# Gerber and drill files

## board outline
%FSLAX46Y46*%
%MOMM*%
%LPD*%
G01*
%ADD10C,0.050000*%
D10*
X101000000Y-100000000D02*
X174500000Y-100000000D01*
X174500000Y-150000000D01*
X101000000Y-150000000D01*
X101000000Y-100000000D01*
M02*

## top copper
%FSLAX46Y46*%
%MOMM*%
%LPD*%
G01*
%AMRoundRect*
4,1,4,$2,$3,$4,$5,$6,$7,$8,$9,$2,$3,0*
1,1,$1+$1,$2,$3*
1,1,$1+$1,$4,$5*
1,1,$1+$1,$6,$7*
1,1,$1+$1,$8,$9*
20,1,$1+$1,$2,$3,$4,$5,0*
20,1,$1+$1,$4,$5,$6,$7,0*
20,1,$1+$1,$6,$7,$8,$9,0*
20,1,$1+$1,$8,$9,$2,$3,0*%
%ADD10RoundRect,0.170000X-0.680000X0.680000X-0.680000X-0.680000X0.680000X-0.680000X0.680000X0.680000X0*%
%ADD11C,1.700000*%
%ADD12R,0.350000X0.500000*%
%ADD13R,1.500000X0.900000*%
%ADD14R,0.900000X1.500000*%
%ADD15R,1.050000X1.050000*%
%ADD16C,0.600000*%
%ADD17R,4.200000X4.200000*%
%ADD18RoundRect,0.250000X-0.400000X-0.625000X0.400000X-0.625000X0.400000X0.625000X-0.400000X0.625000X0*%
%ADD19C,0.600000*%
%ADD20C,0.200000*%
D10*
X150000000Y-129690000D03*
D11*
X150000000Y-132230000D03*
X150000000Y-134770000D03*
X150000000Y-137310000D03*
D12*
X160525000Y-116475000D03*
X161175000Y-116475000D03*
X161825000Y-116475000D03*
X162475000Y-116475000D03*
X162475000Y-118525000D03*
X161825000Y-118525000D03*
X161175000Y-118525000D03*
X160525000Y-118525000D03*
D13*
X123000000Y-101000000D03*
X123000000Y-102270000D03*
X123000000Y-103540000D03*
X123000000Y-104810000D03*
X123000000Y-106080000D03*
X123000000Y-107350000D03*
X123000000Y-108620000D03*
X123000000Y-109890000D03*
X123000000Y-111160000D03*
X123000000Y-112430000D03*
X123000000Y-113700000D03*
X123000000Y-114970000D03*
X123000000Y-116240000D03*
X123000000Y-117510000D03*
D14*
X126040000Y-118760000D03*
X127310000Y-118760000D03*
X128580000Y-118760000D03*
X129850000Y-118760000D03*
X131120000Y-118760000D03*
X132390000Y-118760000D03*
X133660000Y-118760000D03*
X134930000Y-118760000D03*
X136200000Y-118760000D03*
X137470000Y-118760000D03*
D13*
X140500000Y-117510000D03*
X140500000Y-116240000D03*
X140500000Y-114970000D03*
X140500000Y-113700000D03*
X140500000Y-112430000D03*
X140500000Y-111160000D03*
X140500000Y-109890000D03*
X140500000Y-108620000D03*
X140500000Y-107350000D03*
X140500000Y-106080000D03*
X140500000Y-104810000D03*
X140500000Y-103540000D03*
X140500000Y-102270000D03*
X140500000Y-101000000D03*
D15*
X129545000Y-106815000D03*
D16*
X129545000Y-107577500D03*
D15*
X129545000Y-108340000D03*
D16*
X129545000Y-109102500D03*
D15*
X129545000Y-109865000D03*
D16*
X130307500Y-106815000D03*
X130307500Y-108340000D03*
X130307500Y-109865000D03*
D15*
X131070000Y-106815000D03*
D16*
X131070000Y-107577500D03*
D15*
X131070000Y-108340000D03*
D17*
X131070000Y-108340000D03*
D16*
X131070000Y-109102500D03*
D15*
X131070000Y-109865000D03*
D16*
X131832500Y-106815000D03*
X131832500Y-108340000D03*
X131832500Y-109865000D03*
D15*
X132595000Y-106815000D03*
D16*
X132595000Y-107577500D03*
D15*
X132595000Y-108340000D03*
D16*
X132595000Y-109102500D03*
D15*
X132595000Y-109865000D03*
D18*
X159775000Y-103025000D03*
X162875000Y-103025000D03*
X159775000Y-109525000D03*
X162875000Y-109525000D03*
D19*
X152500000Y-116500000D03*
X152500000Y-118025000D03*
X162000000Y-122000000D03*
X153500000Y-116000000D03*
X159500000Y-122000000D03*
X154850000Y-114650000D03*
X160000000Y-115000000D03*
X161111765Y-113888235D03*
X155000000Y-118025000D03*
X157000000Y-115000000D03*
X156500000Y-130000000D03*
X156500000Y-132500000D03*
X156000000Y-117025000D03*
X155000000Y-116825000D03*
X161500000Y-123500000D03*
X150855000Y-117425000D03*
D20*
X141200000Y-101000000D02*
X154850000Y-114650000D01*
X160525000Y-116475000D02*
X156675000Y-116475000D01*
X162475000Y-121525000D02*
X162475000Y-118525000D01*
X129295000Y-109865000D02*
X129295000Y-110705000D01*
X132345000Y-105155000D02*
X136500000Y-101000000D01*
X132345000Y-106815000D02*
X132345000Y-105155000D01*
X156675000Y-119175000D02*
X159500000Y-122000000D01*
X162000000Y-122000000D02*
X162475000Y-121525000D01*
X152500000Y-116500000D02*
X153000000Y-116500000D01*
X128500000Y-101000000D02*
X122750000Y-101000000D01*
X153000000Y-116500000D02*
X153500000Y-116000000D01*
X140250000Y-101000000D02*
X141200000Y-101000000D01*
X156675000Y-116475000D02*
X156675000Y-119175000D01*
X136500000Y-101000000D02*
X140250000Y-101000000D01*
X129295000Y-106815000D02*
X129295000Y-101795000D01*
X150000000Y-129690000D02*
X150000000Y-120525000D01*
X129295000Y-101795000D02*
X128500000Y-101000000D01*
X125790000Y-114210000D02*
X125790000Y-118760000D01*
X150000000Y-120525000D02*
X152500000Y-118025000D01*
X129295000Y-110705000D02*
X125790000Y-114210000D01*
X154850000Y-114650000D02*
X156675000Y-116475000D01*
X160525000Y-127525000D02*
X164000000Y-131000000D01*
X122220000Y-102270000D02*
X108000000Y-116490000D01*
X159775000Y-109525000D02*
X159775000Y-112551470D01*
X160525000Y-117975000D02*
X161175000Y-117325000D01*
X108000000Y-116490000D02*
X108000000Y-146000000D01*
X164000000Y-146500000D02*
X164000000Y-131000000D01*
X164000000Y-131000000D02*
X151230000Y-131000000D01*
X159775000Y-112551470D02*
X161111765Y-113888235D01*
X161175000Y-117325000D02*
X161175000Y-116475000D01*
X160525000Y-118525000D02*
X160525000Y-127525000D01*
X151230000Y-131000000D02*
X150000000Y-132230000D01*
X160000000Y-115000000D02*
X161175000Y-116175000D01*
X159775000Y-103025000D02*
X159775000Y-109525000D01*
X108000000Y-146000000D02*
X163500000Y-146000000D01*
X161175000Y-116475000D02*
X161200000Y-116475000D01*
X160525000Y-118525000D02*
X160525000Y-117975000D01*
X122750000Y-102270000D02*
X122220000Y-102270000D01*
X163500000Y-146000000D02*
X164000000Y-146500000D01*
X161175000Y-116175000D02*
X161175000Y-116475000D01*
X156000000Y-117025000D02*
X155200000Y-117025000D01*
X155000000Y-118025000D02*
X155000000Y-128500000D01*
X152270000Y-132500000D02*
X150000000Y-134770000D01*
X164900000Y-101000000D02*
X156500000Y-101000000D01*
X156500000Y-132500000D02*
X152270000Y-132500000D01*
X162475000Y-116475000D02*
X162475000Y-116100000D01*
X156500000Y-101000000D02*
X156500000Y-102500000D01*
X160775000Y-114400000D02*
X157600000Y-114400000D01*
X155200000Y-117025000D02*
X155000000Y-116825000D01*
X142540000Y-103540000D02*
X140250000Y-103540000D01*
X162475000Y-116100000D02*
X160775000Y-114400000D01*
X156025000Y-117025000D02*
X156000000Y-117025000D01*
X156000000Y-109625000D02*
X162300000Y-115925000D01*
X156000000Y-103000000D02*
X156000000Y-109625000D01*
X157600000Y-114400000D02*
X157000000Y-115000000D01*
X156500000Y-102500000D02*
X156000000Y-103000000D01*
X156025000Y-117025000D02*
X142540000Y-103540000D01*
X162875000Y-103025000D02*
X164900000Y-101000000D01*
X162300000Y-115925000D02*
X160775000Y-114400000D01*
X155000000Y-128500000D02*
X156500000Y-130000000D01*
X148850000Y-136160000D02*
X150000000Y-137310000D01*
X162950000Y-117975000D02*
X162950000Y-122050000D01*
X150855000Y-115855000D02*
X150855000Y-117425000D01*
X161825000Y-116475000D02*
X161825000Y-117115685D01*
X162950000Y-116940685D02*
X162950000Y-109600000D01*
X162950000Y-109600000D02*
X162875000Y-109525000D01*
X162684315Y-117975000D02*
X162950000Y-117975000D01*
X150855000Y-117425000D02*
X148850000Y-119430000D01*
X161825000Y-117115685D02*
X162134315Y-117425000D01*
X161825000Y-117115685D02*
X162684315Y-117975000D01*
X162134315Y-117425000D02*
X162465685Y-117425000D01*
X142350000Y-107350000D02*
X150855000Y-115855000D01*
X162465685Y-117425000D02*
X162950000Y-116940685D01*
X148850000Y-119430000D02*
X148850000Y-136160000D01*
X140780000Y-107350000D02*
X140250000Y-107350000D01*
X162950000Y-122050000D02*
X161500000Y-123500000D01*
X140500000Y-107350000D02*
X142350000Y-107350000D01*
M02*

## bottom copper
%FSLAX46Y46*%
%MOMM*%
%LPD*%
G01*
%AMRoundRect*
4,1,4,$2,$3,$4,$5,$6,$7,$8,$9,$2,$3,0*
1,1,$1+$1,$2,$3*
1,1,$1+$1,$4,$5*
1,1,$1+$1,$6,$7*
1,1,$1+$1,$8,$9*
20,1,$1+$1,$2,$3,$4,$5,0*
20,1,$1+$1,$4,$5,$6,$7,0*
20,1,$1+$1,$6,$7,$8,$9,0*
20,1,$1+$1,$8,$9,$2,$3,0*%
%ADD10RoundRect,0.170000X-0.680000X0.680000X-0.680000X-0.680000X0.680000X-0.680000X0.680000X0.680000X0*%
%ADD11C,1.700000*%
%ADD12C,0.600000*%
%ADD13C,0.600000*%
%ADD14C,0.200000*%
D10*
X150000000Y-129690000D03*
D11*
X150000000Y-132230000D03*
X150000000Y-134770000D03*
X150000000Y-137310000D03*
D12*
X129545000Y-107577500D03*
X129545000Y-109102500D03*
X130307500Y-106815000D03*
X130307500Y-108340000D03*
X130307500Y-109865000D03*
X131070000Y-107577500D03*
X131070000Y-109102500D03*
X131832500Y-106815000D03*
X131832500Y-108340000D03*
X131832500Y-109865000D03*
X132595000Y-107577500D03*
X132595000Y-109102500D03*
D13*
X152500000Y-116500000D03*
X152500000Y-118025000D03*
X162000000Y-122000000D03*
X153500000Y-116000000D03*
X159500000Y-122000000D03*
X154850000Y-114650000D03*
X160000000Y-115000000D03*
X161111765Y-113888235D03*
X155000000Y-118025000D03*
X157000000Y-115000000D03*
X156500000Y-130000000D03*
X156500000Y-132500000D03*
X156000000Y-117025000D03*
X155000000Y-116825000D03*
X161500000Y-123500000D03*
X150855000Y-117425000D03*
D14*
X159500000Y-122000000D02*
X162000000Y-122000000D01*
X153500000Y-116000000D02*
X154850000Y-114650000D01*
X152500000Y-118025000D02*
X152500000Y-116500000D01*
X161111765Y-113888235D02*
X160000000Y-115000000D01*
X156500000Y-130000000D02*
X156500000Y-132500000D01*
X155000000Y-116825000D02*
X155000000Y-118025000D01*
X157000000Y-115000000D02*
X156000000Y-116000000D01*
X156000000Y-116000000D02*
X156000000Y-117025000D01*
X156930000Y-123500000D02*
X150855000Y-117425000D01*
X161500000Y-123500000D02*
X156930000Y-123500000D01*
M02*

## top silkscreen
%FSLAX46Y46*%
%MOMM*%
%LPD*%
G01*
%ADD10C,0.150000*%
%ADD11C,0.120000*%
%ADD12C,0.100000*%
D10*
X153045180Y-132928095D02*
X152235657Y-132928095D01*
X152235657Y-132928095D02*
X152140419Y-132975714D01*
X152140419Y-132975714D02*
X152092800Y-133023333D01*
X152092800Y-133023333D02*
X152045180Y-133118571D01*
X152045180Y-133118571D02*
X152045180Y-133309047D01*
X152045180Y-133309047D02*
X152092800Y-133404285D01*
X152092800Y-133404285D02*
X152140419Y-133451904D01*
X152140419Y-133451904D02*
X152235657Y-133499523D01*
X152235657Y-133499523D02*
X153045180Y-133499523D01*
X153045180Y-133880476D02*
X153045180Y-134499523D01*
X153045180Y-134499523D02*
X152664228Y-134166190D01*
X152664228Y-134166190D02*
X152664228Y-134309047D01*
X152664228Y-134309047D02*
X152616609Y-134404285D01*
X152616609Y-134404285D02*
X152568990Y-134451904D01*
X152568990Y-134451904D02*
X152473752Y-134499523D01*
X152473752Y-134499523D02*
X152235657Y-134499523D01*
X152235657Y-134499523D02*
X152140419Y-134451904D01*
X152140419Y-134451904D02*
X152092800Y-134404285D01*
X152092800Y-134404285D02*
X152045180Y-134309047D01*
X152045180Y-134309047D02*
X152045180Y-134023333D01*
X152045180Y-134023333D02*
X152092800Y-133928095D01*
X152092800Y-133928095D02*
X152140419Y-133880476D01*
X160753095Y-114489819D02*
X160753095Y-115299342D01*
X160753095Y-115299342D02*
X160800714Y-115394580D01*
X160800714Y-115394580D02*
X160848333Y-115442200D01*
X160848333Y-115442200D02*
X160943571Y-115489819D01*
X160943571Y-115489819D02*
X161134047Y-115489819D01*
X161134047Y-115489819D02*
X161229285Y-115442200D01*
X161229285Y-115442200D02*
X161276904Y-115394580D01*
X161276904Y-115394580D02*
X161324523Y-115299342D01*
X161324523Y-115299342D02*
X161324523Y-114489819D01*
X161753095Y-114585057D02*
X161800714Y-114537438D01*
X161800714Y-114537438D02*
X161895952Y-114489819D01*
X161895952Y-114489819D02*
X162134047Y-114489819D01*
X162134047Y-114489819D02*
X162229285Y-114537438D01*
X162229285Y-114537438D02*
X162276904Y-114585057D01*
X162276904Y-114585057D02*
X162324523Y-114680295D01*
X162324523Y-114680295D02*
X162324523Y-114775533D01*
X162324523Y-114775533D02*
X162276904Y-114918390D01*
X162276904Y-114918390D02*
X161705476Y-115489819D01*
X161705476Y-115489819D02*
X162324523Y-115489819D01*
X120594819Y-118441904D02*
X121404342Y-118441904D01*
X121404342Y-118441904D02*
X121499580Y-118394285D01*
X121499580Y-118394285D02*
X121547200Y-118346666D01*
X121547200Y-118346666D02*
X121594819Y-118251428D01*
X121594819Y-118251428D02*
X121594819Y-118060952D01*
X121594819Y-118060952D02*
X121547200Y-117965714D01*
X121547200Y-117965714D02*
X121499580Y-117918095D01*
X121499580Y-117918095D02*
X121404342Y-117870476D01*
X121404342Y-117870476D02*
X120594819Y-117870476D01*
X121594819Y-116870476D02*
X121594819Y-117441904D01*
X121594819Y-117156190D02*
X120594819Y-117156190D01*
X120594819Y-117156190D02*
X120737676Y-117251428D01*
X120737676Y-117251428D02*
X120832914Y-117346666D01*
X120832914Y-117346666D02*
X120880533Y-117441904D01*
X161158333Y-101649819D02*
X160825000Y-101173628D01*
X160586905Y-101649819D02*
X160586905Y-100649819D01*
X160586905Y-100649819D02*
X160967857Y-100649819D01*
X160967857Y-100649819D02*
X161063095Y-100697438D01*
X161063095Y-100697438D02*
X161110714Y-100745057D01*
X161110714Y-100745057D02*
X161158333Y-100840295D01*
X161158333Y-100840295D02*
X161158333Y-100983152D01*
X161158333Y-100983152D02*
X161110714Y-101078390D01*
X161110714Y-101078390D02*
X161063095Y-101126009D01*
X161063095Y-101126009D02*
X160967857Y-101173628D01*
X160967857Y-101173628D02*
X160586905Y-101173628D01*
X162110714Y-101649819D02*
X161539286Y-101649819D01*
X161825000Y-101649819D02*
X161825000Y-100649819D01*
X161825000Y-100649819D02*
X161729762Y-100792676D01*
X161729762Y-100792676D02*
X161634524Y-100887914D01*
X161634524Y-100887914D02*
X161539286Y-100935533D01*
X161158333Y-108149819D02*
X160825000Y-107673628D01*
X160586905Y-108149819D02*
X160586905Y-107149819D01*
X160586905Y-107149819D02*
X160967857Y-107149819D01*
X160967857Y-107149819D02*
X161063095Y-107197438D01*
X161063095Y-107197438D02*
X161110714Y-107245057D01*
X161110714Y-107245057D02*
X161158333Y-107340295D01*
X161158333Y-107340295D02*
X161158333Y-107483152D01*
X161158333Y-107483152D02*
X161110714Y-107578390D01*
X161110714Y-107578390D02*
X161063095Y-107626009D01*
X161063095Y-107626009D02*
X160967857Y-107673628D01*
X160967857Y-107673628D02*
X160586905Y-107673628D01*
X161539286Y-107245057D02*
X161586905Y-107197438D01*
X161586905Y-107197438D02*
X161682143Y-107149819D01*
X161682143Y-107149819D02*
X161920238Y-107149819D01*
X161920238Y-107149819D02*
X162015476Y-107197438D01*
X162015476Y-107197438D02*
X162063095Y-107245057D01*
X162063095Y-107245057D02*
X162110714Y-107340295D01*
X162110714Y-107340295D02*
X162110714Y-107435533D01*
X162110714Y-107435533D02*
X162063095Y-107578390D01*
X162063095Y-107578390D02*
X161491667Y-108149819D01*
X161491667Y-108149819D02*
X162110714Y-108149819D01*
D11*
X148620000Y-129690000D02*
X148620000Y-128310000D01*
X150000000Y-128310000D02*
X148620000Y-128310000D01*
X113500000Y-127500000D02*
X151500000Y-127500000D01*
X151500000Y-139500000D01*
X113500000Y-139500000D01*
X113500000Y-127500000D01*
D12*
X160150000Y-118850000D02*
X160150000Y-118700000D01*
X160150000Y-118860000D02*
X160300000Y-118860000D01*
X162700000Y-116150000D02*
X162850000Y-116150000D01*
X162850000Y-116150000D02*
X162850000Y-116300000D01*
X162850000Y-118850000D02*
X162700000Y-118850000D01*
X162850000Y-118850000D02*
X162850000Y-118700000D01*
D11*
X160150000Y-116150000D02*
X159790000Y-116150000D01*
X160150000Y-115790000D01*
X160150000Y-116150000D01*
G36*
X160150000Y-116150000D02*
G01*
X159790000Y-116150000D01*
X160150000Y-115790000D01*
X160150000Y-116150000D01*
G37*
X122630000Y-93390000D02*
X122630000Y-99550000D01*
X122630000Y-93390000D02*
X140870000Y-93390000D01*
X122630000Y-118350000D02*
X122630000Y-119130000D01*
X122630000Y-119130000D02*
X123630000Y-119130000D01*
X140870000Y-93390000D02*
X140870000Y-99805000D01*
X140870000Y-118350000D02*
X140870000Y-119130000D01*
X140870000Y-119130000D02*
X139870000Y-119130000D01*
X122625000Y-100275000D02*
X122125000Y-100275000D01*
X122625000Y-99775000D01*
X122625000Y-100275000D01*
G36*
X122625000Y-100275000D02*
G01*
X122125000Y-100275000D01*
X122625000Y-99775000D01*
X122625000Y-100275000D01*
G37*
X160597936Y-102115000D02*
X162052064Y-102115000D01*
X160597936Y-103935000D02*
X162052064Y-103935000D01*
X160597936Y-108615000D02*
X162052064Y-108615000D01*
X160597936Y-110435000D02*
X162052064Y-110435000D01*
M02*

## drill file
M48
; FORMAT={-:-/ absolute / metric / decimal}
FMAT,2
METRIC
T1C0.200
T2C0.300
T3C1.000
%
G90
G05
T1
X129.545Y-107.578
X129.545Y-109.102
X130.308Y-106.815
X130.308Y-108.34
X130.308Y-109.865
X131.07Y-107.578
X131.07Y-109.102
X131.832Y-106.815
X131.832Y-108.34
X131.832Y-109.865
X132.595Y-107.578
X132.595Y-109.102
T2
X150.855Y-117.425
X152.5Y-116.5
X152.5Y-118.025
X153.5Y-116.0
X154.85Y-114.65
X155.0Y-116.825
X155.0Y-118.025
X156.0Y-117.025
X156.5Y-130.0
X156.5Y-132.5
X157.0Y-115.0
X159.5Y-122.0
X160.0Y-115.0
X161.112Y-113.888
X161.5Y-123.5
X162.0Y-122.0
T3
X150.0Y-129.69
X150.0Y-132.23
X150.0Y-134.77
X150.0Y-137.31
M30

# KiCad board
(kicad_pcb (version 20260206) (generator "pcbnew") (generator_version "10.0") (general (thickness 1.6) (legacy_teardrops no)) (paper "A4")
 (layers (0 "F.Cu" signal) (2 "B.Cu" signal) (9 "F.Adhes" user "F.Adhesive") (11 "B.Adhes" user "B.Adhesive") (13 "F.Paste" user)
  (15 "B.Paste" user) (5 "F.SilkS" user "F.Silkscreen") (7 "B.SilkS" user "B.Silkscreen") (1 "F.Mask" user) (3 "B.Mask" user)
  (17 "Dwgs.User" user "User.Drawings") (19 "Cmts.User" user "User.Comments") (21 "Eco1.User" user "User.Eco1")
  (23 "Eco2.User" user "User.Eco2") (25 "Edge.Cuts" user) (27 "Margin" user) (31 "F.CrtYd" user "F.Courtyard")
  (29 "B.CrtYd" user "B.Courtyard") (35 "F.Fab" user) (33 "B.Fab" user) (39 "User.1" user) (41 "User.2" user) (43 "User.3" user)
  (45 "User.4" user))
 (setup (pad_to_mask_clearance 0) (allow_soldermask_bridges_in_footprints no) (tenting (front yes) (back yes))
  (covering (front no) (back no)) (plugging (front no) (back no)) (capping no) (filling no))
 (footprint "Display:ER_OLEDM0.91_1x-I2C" (layer "F.Cu") (at 150 129.69 -90)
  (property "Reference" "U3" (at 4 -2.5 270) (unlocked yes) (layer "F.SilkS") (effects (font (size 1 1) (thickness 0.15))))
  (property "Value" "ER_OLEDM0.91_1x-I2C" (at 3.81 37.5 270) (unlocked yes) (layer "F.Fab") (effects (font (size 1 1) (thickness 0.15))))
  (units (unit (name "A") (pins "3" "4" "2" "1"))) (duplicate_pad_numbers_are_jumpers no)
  (fp_line (start 0 1.38) (end -1.38 1.38) (stroke (width 0.12) (type solid)) (layer "F.SilkS"))
  (fp_line (start -1.38 0) (end -1.38 1.38) (stroke (width 0.12) (type solid)) (layer "F.SilkS"))
  (fp_rect (start -2.19 -1.5) (end 9.81 36.5) (stroke (width 0.12) (type solid)) (fill no) (layer "F.SilkS"))
  (pad "1" thru_hole roundrect (at 0 0 270) (size 1.7 1.7) (drill 1) (layers "*.Cu" "*.Mask") (remove_unused_layers no)
   (roundrect_rratio 0.1) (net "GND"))
  (pad "2" thru_hole circle (at 2.54 0 270) (size 1.7 1.7) (drill 1) (layers "*.Cu" "*.Mask") (remove_unused_layers no) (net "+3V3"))
  (pad "3" thru_hole circle (at 5.08 0 270) (size 1.7 1.7) (drill 1) (layers "*.Cu" "*.Mask") (remove_unused_layers no)
   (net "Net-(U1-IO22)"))
  (pad "4" thru_hole circle (at 7.62 0 270) (size 1.7 1.7) (drill 1) (layers "*.Cu" "*.Mask") (remove_unused_layers no)
   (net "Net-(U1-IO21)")))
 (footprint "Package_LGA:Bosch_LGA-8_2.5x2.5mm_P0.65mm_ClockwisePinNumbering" (layer "F.Cu") (at 161.5 117.5)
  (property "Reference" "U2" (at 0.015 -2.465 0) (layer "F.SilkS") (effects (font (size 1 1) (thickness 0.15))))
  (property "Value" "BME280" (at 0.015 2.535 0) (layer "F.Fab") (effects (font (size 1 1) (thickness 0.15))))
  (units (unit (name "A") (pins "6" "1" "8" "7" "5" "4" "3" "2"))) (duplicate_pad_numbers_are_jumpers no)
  (fp_line (start -1.35 1.35) (end -1.35 1.2) (stroke (width 0.1) (type solid)) (layer "F.SilkS"))
  (fp_line (start -1.35 1.36) (end -1.2 1.36) (stroke (width 0.1) (type solid)) (layer "F.SilkS"))
  (fp_line (start 1.2 -1.35) (end 1.35 -1.35) (stroke (width 0.1) (type solid)) (layer "F.SilkS"))
  (fp_line (start 1.35 -1.35) (end 1.35 -1.2) (stroke (width 0.1) (type solid)) (layer "F.SilkS"))
  (fp_line (start 1.35 1.35) (end 1.2 1.35) (stroke (width 0.1) (type solid)) (layer "F.SilkS"))
  (fp_line (start 1.35 1.35) (end 1.35 1.2) (stroke (width 0.1) (type solid)) (layer "F.SilkS"))
  (fp_poly
   (pts (xy -1.35 -1.35) (xy -1.71 -1.35) (xy -1.35 -1.71) (xy -1.35 -1.35)) (stroke (width 0.12) (type solid)) (fill yes) (layer "F.SilkS"))
  (pad "1" smd rect (at -0.975 -1.025 90) (size 0.5 0.35) (layers "F.Cu" "F.Mask" "F.Paste") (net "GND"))
  (pad "2" smd rect (at -0.325 -1.025 90) (size 0.5 0.35) (layers "F.Cu" "F.Mask" "F.Paste") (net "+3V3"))
  (pad "3" smd rect (at 0.325 -1.025 90) (size 0.5 0.35) (layers "F.Cu" "F.Mask" "F.Paste") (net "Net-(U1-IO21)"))
  (pad "4" smd rect (at 0.975 -1.025 90) (size 0.5 0.35) (layers "F.Cu" "F.Mask" "F.Paste") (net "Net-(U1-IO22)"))
  (pad "5" smd rect (at 0.975 1.025 90) (size 0.5 0.35) (layers "F.Cu" "F.Mask" "F.Paste") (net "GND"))
  (pad "6" smd rect (at 0.325 1.025 90) (size 0.5 0.35) (layers "F.Cu" "F.Mask" "F.Paste") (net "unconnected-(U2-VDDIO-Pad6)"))
  (pad "7" smd rect (at -0.325 1.025 90) (size 0.5 0.35) (layers "F.Cu" "F.Mask" "F.Paste") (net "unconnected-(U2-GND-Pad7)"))
  (pad "8" smd rect (at -0.975 1.025 90) (size 0.5 0.35) (layers "F.Cu" "F.Mask" "F.Paste") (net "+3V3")))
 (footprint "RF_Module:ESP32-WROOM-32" (layer "F.Cu") (at 131.75 109.25)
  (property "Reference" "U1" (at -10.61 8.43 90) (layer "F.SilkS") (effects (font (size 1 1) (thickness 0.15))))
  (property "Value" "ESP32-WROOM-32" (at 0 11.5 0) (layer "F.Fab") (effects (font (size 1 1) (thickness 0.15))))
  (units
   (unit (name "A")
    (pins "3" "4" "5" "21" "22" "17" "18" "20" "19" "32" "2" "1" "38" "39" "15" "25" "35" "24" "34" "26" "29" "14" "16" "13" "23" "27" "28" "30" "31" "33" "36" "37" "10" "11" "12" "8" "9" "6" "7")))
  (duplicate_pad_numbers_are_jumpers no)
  (fp_line (start -9.12 -15.86) (end -9.12 -9.7) (stroke (width 0.12) (type solid)) (layer "F.SilkS"))
  (fp_line (start -9.12 -15.86) (end 9.12 -15.86) (stroke (width 0.12) (type solid)) (layer "F.SilkS"))
  (fp_line (start -9.12 9.1) (end -9.12 9.88) (stroke (width 0.12) (type solid)) (layer "F.SilkS"))
  (fp_line (start -9.12 9.88) (end -8.12 9.88) (stroke (width 0.12) (type solid)) (layer "F.SilkS"))
  (fp_line (start 9.12 -15.86) (end 9.12 -9.445) (stroke (width 0.12) (type solid)) (layer "F.SilkS"))
  (fp_line (start 9.12 9.1) (end 9.12 9.88) (stroke (width 0.12) (type solid)) (layer "F.SilkS"))
  (fp_line (start 9.12 9.88) (end 8.12 9.88) (stroke (width 0.12) (type solid)) (layer "F.SilkS"))
  (fp_poly
   (pts (xy -9.125 -8.975) (xy -9.625 -8.975) (xy -9.125 -9.475) (xy -9.125 -8.975)) (stroke (width 0.12) (type solid)) (fill yes)
   (layer "F.SilkS"))
  (pad "1" smd rect (at -8.75 -8.25) (size 1.5 0.9) (layers "F.Cu" "F.Mask" "F.Paste") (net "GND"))
  (pad "2" smd rect (at -8.75 -6.98) (size 1.5 0.9) (layers "F.Cu" "F.Mask" "F.Paste") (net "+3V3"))
  (pad "3" smd rect (at -8.75 -5.71) (size 1.5 0.9) (layers "F.Cu" "F.Mask" "F.Paste") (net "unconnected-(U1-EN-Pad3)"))
  (pad "4" smd rect (at -8.75 -4.44) (size 1.5 0.9) (layers "F.Cu" "F.Mask" "F.Paste") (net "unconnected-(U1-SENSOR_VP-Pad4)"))
  (pad "5" smd rect (at -8.75 -3.17) (size 1.5 0.9) (layers "F.Cu" "F.Mask" "F.Paste") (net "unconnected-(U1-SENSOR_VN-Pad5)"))
  (pad "6" smd rect (at -8.75 -1.9) (size 1.5 0.9) (layers "F.Cu" "F.Mask" "F.Paste") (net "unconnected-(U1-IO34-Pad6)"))
  (pad "7" smd rect (at -8.75 -0.63) (size 1.5 0.9) (layers "F.Cu" "F.Mask" "F.Paste") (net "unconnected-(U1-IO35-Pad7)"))
  (pad "8" smd rect (at -8.75 0.64) (size 1.5 0.9) (layers "F.Cu" "F.Mask" "F.Paste") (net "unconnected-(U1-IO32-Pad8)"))
  (pad "9" smd rect (at -8.75 1.91) (size 1.5 0.9) (layers "F.Cu" "F.Mask" "F.Paste") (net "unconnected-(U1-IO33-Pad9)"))
  (pad "10" smd rect (at -8.75 3.18) (size 1.5 0.9) (layers "F.Cu" "F.Mask" "F.Paste") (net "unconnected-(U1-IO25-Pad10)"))
  (pad "11" smd rect (at -8.75 4.45) (size 1.5 0.9) (layers "F.Cu" "F.Mask" "F.Paste") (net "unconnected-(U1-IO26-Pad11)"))
  (pad "12" smd rect (at -8.75 5.72) (size 1.5 0.9) (layers "F.Cu" "F.Mask" "F.Paste") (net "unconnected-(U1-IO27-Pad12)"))
  (pad "13" smd rect (at -8.75 6.99) (size 1.5 0.9) (layers "F.Cu" "F.Mask" "F.Paste") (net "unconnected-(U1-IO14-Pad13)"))
  (pad "14" smd rect (at -8.75 8.26) (size 1.5 0.9) (layers "F.Cu" "F.Mask" "F.Paste") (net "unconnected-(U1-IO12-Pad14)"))
  (pad "15" smd rect (at -5.71 9.51 90) (size 1.5 0.9) (layers "F.Cu" "F.Mask" "F.Paste") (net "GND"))
  (pad "16" smd rect (at -4.44 9.51 90) (size 1.5 0.9) (layers "F.Cu" "F.Mask" "F.Paste") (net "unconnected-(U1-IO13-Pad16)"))
  (pad "17" smd rect (at -3.17 9.51 90) (size 1.5 0.9) (layers "F.Cu" "F.Mask" "F.Paste") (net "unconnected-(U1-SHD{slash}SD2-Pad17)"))
  (pad "18" smd rect (at -1.9 9.51 90) (size 1.5 0.9) (layers "F.Cu" "F.Mask" "F.Paste") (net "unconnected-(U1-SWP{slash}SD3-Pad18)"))
  (pad "19" smd rect (at -0.63 9.51 90) (size 1.5 0.9) (layers "F.Cu" "F.Mask" "F.Paste") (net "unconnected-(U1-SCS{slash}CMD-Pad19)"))
  (pad "20" smd rect (at 0.64 9.51 90) (size 1.5 0.9) (layers "F.Cu" "F.Mask" "F.Paste") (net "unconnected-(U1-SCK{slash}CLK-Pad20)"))
  (pad "21" smd rect (at 1.91 9.51 90) (size 1.5 0.9) (layers "F.Cu" "F.Mask" "F.Paste") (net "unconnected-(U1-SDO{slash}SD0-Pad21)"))
  (pad "22" smd rect (at 3.18 9.51 90) (size 1.5 0.9) (layers "F.Cu" "F.Mask" "F.Paste") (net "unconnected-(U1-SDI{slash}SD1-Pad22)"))
  (pad "23" smd rect (at 4.45 9.51 90) (size 1.5 0.9) (layers "F.Cu" "F.Mask" "F.Paste") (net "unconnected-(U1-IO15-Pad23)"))
  (pad "24" smd rect (at 5.72 9.51 90) (size 1.5 0.9) (layers "F.Cu" "F.Mask" "F.Paste") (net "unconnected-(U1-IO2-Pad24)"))
  (pad "25" smd rect (at 8.75 8.26) (size 1.5 0.9) (layers "F.Cu" "F.Mask" "F.Paste") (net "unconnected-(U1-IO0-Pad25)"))
  (pad "26" smd rect (at 8.75 6.99) (size 1.5 0.9) (layers "F.Cu" "F.Mask" "F.Paste") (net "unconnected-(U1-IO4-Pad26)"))
  (pad "27" smd rect (at 8.75 5.72) (size 1.5 0.9) (layers "F.Cu" "F.Mask" "F.Paste") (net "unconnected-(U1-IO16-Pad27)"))
  (pad "28" smd rect (at 8.75 4.45) (size 1.5 0.9) (layers "F.Cu" "F.Mask" "F.Paste") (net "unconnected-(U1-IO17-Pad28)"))
  (pad "29" smd rect (at 8.75 3.18) (size 1.5 0.9) (layers "F.Cu" "F.Mask" "F.Paste") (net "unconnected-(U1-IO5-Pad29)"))
  (pad "30" smd rect (at 8.75 1.91) (size 1.5 0.9) (layers "F.Cu" "F.Mask" "F.Paste") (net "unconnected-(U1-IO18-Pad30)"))
  (pad "31" smd rect (at 8.75 0.64) (size 1.5 0.9) (layers "F.Cu" "F.Mask" "F.Paste") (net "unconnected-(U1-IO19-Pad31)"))
  (pad "32" smd rect (at 8.75 -0.63) (size 1.5 0.9) (layers "F.Cu" "F.Mask" "F.Paste") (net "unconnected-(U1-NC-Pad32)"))
  (pad "33" smd rect (at 8.75 -1.9) (size 1.5 0.9) (layers "F.Cu" "F.Mask" "F.Paste") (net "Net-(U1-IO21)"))
  (pad "34" smd rect (at 8.75 -3.17) (size 1.5 0.9) (layers "F.Cu" "F.Mask" "F.Paste") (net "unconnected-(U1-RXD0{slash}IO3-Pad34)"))
  (pad "35" smd rect (at 8.75 -4.44) (size 1.5 0.9) (layers "F.Cu" "F.Mask" "F.Paste") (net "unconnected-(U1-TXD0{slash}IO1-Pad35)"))
  (pad "36" smd rect (at 8.75 -5.71) (size 1.5 0.9) (layers "F.Cu" "F.Mask" "F.Paste") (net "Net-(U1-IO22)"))
  (pad "37" smd rect (at 8.75 -6.98) (size 1.5 0.9) (layers "F.Cu" "F.Mask" "F.Paste") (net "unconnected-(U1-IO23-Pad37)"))
  (pad "38" smd rect (at 8.75 -8.25) (size 1.5 0.9) (layers "F.Cu" "F.Mask" "F.Paste") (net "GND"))
  (pad "39" smd rect (at -2.205 -2.435) (size 1.05 1.05) (layers "F.Cu" "F.Paste") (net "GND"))
  (pad "39" thru_hole circle (at -2.205 -1.6725) (size 0.6 0.6) (drill 0.2) (layers "*.Cu" "F.Mask") (remove_unused_layers no) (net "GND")
   (zone_connect 2))
  (pad "39" smd rect (at -2.205 -0.91) (size 1.05 1.05) (layers "F.Cu" "F.Paste") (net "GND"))
  (pad "39" thru_hole circle (at -2.205 -0.1475) (size 0.6 0.6) (drill 0.2) (layers "*.Cu" "F.Mask") (remove_unused_layers no) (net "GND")
   (zone_connect 2))
  (pad "39" smd rect (at -2.205 0.615) (size 1.05 1.05) (layers "F.Cu" "F.Paste") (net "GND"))
  (pad "39" thru_hole circle (at -1.4425 -2.435) (size 0.6 0.6) (drill 0.2) (layers "*.Cu" "F.Mask") (remove_unused_layers no) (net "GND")
   (zone_connect 2))
  (pad "39" thru_hole circle (at -1.4425 -0.91) (size 0.6 0.6) (drill 0.2) (layers "*.Cu" "F.Mask") (remove_unused_layers no) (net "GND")
   (zone_connect 2))
  (pad "39" thru_hole circle (at -1.4425 0.615) (size 0.6 0.6) (drill 0.2) (layers "*.Cu" "F.Mask") (remove_unused_layers no) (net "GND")
   (zone_connect 2))
  (pad "39" smd rect (at -0.68 -2.435) (size 1.05 1.05) (layers "F.Cu" "F.Paste") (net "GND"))
  (pad "39" thru_hole circle (at -0.68 -1.6725) (size 0.6 0.6) (drill 0.2) (layers "*.Cu" "F.Mask") (remove_unused_layers no) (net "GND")
   (zone_connect 2))
  (pad "39" smd rect (at -0.68 -0.91) (size 1.05 1.05) (layers "F.Cu" "F.Paste") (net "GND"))
  (pad "39" smd rect (at -0.68 -0.91) (size 4.2 4.2) (layers "F.Cu" "F.Mask") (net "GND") (zone_connect 2))
  (pad "39" thru_hole circle (at -0.68 -0.1475) (size 0.6 0.6) (drill 0.2) (layers "*.Cu" "F.Mask") (remove_unused_layers no) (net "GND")
   (zone_connect 2))
  (pad "39" smd rect (at -0.68 0.615) (size 1.05 1.05) (layers "F.Cu" "F.Paste") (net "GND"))
  (pad "39" thru_hole circle (at 0.0825 -2.435) (size 0.6 0.6) (drill 0.2) (layers "*.Cu" "F.Mask") (remove_unused_layers no) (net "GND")
   (zone_connect 2))
  (pad "39" thru_hole circle (at 0.0825 -0.91) (size 0.6 0.6) (drill 0.2) (layers "*.Cu" "F.Mask") (remove_unused_layers no) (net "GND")
   (zone_connect 2))
  (pad "39" thru_hole circle (at 0.0825 0.615) (size 0.6 0.6) (drill 0.2) (layers "*.Cu" "F.Mask") (remove_unused_layers no) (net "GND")
   (zone_connect 2))
  (pad "39" smd rect (at 0.845 -2.435) (size 1.05 1.05) (layers "F.Cu" "F.Paste") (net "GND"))
  (pad "39" thru_hole circle (at 0.845 -1.6725) (size 0.6 0.6) (drill 0.2) (layers "*.Cu" "F.Mask") (remove_unused_layers no) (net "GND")
   (zone_connect 2))
  (pad "39" smd rect (at 0.845 -0.91) (size 1.05 1.05) (layers "F.Cu" "F.Paste") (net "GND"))
  (pad "39" thru_hole circle (at 0.845 -0.1475) (size 0.6 0.6) (drill 0.2) (layers "*.Cu" "F.Mask") (remove_unused_layers no) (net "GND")
   (zone_connect 2))
  (pad "39" smd rect (at 0.845 0.615) (size 1.05 1.05) (layers "F.Cu" "F.Paste") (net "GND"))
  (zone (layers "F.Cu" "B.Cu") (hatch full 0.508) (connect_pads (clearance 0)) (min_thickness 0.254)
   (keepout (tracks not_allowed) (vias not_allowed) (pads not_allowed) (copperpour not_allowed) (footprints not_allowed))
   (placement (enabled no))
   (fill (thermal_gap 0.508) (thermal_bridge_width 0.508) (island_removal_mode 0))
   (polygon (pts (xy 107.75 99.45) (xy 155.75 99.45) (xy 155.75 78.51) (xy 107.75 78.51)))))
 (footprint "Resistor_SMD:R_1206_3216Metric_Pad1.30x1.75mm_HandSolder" (layer "F.Cu") (at 161.325 103.025)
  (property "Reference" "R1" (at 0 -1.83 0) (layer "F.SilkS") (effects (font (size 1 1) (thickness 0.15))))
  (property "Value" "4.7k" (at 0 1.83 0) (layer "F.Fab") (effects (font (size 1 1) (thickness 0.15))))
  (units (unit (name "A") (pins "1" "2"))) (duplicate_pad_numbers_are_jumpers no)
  (fp_line (start -0.727064 -0.91) (end 0.727064 -0.91) (stroke (width 0.12) (type solid)) (layer "F.SilkS"))
  (fp_line (start -0.727064 0.91) (end 0.727064 0.91) (stroke (width 0.12) (type solid)) (layer "F.SilkS"))
  (pad "1" smd roundrect (at -1.55 0) (size 1.3 1.75) (layers "F.Cu" "F.Mask" "F.Paste") (roundrect_rratio 0.192308) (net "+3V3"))
  (pad "2" smd roundrect (at 1.55 0) (size 1.3 1.75) (layers "F.Cu" "F.Mask" "F.Paste") (roundrect_rratio 0.192308) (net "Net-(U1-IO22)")))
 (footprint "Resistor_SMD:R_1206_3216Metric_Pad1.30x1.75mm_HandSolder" (layer "F.Cu") (at 161.325 109.525)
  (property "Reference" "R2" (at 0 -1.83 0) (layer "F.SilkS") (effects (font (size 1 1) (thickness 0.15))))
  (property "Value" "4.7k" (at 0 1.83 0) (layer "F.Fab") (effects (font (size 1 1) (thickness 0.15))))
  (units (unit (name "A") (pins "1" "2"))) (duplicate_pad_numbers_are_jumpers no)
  (fp_line (start -0.727064 -0.91) (end 0.727064 -0.91) (stroke (width 0.12) (type solid)) (layer "F.SilkS"))
  (fp_line (start -0.727064 0.91) (end 0.727064 0.91) (stroke (width 0.12) (type solid)) (layer "F.SilkS"))
  (pad "1" smd roundrect (at -1.55 0) (size 1.3 1.75) (layers "F.Cu" "F.Mask" "F.Paste") (roundrect_rratio 0.192308) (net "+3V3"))
  (pad "2" smd roundrect (at 1.55 0) (size 1.3 1.75) (layers "F.Cu" "F.Mask" "F.Paste") (roundrect_rratio 0.192308) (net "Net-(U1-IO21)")))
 (gr_rect (start 101 100) (end 174.5 150) (stroke (width 0.05) (type default)) (fill no) (layer "Edge.Cuts"))
 (segment (start 141.2 101) (end 154.85 114.65) (width 0.2) (layer "F.Cu") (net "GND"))
 (segment (start 160.525 116.475) (end 156.675 116.475) (width 0.2) (layer "F.Cu") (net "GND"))
 (segment (start 162.475 121.525) (end 162.475 118.525) (width 0.2) (layer "F.Cu") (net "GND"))
 (segment (start 129.295 109.865) (end 129.295 110.705) (width 0.2) (layer "F.Cu") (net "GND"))
 (segment (start 132.345 105.155) (end 136.5 101) (width 0.2) (layer "F.Cu") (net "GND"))
 (segment (start 132.345 106.815) (end 132.345 105.155) (width 0.2) (layer "F.Cu") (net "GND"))
 (segment (start 156.675 119.175) (end 159.5 122) (width 0.2) (layer "F.Cu") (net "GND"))
 (segment (start 162 122) (end 162.475 121.525) (width 0.2) (layer "F.Cu") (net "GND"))
 (segment (start 152.5 116.5) (end 153 116.5) (width 0.2) (layer "F.Cu") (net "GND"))
 (segment (start 128.5 101) (end 122.75 101) (width 0.2) (layer "F.Cu") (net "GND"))
 (segment (start 153 116.5) (end 153.5 116) (width 0.2) (layer "F.Cu") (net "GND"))
 (segment (start 140.25 101) (end 141.2 101) (width 0.2) (layer "F.Cu") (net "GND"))
 (segment (start 156.675 116.475) (end 156.675 119.175) (width 0.2) (layer "F.Cu") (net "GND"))
 (segment (start 136.5 101) (end 140.25 101) (width 0.2) (layer "F.Cu") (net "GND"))
 (segment (start 129.295 106.815) (end 129.295 101.795) (width 0.2) (layer "F.Cu") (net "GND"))
 (segment (start 150 129.69) (end 150 120.525) (width 0.2) (layer "F.Cu") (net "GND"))
 (segment (start 129.295 101.795) (end 128.5 101) (width 0.2) (layer "F.Cu") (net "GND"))
 (segment (start 125.79 114.21) (end 125.79 118.76) (width 0.2) (layer "F.Cu") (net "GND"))
 (segment (start 150 120.525) (end 152.5 118.025) (width 0.2) (layer "F.Cu") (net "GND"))
 (segment (start 129.295 110.705) (end 125.79 114.21) (width 0.2) (layer "F.Cu") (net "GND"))
 (segment (start 154.85 114.65) (end 156.675 116.475) (width 0.2) (layer "F.Cu") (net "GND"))
 (via (at 152.5 116.5) (size 0.6) (drill 0.3) (layers "F.Cu" "B.Cu") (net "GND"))
 (via (at 152.5 118.025) (size 0.6) (drill 0.3) (layers "F.Cu" "B.Cu") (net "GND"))
 (via (at 162 122) (size 0.6) (drill 0.3) (layers "F.Cu" "B.Cu") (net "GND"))
 (via (at 153.5 116) (size 0.6) (drill 0.3) (layers "F.Cu" "B.Cu") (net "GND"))
 (via (at 159.5 122) (size 0.6) (drill 0.3) (layers "F.Cu" "B.Cu") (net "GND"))
 (via (at 154.85 114.65) (size 0.6) (drill 0.3) (layers "F.Cu" "B.Cu") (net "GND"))
 (segment (start 159.5 122) (end 162 122) (width 0.2) (layer "B.Cu") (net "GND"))
 (segment (start 153.5 116) (end 154.85 114.65) (width 0.2) (layer "B.Cu") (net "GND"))
 (segment (start 152.5 118.025) (end 152.5 116.5) (width 0.2) (layer "B.Cu") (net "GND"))
 (segment (start 160.525 127.525) (end 164 131) (width 0.2) (layer "F.Cu") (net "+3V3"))
 (segment (start 122.22 102.27) (end 108 116.49) (width 0.2) (layer "F.Cu") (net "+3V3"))
 (segment (start 159.775 109.525) (end 159.775 112.55147) (width 0.2) (layer "F.Cu") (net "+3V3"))
 (segment (start 160.525 117.975) (end 161.175 117.325) (width 0.2) (layer "F.Cu") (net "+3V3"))
 (segment (start 108 116.49) (end 108 146) (width 0.2) (layer "F.Cu") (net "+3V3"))
 (segment (start 164 146.5) (end 164 131) (width 0.2) (layer "F.Cu") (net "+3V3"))
 (segment (start 164 131) (end 151.23 131) (width 0.2) (layer "F.Cu") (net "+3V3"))
 (segment (start 159.775 112.55147) (end 161.111765 113.888235) (width 0.2) (layer "F.Cu") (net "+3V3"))
 (segment (start 161.175 117.325) (end 161.175 116.475) (width 0.2) (layer "F.Cu") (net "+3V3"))
 (segment (start 160.525 118.525) (end 160.525 127.525) (width 0.2) (layer "F.Cu") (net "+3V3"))
 (segment (start 151.23 131) (end 150 132.23) (width 0.2) (layer "F.Cu") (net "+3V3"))
 (segment (start 160 115) (end 161.175 116.175) (width 0.2) (layer "F.Cu") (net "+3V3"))
 (segment (start 159.775 103.025) (end 159.775 109.525) (width 0.2) (layer "F.Cu") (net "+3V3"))
 (segment (start 108 146) (end 163.5 146) (width 0.2) (layer "F.Cu") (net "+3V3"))
 (segment (start 161.175 116.475) (end 161.2 116.475) (width 0.2) (layer "F.Cu") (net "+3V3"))
 (segment (start 160.525 118.525) (end 160.525 117.975) (width 0.2) (layer "F.Cu") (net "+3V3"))
 (segment (start 122.75 102.27) (end 122.22 102.27) (width 0.2) (layer "F.Cu") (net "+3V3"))
 (segment (start 163.5 146) (end 164 146.5) (width 0.2) (layer "F.Cu") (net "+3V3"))
 (segment (start 161.175 116.175) (end 161.175 116.475) (width 0.2) (layer "F.Cu") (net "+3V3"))
 (via (at 160 115) (size 0.6) (drill 0.3) (layers "F.Cu" "B.Cu") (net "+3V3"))
 (via (at 161.111765 113.888235) (size 0.6) (drill 0.3) (layers "F.Cu" "B.Cu") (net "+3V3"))
 (segment (start 161.111765 113.888235) (end 160 115) (width 0.2) (layer "B.Cu") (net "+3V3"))
 (segment (start 156 117.025) (end 155.2 117.025) (width 0.2) (layer "F.Cu") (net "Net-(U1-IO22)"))
 (segment (start 155 118.025) (end 155 128.5) (width 0.2) (layer "F.Cu") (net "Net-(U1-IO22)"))
 (segment (start 152.27 132.5) (end 150 134.77) (width 0.2) (layer "F.Cu") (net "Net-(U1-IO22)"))
 (segment (start 164.9 101) (end 156.5 101) (width 0.2) (layer "F.Cu") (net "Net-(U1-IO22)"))
 (segment (start 156.5 132.5) (end 152.27 132.5) (width 0.2) (layer "F.Cu") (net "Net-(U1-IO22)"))
 (segment (start 162.475 116.475) (end 162.475 116.1) (width 0.2) (layer "F.Cu") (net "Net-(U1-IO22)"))
 (segment (start 156.5 101) (end 156.5 102.5) (width 0.2) (layer "F.Cu") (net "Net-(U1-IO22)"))
 (segment (start 160.775 114.4) (end 157.6 114.4) (width 0.2) (layer "F.Cu") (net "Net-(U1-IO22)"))
 (segment (start 155.2 117.025) (end 155 116.825) (width 0.2) (layer "F.Cu") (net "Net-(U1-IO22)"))
 (segment (start 142.54 103.54) (end 140.25 103.54) (width 0.2) (layer "F.Cu") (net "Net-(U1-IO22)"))
 (segment (start 162.475 116.1) (end 160.775 114.4) (width 0.2) (layer "F.Cu") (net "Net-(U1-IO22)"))
 (segment (start 156.025 117.025) (end 156 117.025) (width 0.2) (layer "F.Cu") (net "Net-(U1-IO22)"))
 (segment (start 156 109.625) (end 162.3 115.925) (width 0.2) (layer "F.Cu") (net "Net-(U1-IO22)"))
 (segment (start 156 103) (end 156 109.625) (width 0.2) (layer "F.Cu") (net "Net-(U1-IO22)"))
 (segment (start 157.6 114.4) (end 157 115) (width 0.2) (layer "F.Cu") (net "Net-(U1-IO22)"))
 (segment (start 156.5 102.5) (end 156 103) (width 0.2) (layer "F.Cu") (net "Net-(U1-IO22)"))
 (segment (start 156.025 117.025) (end 142.54 103.54) (width 0.2) (layer "F.Cu") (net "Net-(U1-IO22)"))
 (segment (start 162.875 103.025) (end 164.9 101) (width 0.2) (layer "F.Cu") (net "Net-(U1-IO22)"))
 (segment (start 162.3 115.925) (end 160.775 114.4) (width 0.2) (layer "F.Cu") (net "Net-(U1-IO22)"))
 (segment (start 155 128.5) (end 156.5 130) (width 0.2) (layer "F.Cu") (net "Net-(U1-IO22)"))
 (via (at 155 118.025) (size 0.6) (drill 0.3) (layers "F.Cu" "B.Cu") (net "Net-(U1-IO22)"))
 (via (at 157 115) (size 0.6) (drill 0.3) (layers "F.Cu" "B.Cu") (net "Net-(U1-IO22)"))
 (via (at 156.5 130) (size 0.6) (drill 0.3) (layers "F.Cu" "B.Cu") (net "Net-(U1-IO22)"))
 (via (at 156.5 132.5) (size 0.6) (drill 0.3) (layers "F.Cu" "B.Cu") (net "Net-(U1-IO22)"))
 (via (at 156 117.025) (size 0.6) (drill 0.3) (layers "F.Cu" "B.Cu") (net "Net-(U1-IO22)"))
 (via (at 155 116.825) (size 0.6) (drill 0.3) (layers "F.Cu" "B.Cu") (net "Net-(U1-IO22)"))
 (segment (start 156.5 130) (end 156.5 132.5) (width 0.2) (layer "B.Cu") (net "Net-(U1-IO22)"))
 (segment (start 155 116.825) (end 155 118.025) (width 0.2) (layer "B.Cu") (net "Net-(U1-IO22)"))
 (segment (start 157 115) (end 156 116) (width 0.2) (layer "B.Cu") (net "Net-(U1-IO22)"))
 (segment (start 156 116) (end 156 117.025) (width 0.2) (layer "B.Cu") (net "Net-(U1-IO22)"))
 (segment (start 148.85 136.16) (end 150 137.31) (width 0.2) (layer "F.Cu") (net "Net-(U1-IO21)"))
 (segment (start 162.95 117.975) (end 162.95 122.05) (width 0.2) (layer "F.Cu") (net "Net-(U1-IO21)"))
 (segment (start 150.855 115.855) (end 150.855 117.425) (width 0.2) (layer "F.Cu") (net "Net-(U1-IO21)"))
 (segment (start 161.825 116.475) (end 161.825 117.115685) (width 0.2) (layer "F.Cu") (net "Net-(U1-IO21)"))
 (segment (start 162.95 116.940685) (end 162.95 109.6) (width 0.2) (layer "F.Cu") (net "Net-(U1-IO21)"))
 (segment (start 162.95 109.6) (end 162.875 109.525) (width 0.2) (layer "F.Cu") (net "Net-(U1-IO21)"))
 (segment (start 162.684315 117.975) (end 162.95 117.975) (width 0.2) (layer "F.Cu") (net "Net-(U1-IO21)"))
 (segment (start 150.855 117.425) (end 148.85 119.43) (width 0.2) (layer "F.Cu") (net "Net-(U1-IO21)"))
 (segment (start 161.825 117.115685) (end 162.134315 117.425) (width 0.2) (layer "F.Cu") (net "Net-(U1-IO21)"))
 (segment (start 161.825 117.115685) (end 162.684315 117.975) (width 0.2) (layer "F.Cu") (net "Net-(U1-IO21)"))
 (segment (start 162.134315 117.425) (end 162.465685 117.425) (width 0.2) (layer "F.Cu") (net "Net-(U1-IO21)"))
 (segment (start 142.35 107.35) (end 150.855 115.855) (width 0.2) (layer "F.Cu") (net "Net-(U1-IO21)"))
 (segment (start 162.465685 117.425) (end 162.95 116.940685) (width 0.2) (layer "F.Cu") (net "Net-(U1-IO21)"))
 (segment (start 148.85 119.43) (end 148.85 136.16) (width 0.2) (layer "F.Cu") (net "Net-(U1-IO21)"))
 (segment (start 140.78 107.35) (end 140.25 107.35) (width 0.2) (layer "F.Cu") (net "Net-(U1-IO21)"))
 (segment (start 162.95 122.05) (end 161.5 123.5) (width 0.2) (layer "F.Cu") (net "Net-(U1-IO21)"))
 (segment (start 140.5 107.35) (end 142.35 107.35) (width 0.2) (layer "F.Cu") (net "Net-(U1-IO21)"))
 (via (at 161.5 123.5) (size 0.6) (drill 0.3) (layers "F.Cu" "B.Cu") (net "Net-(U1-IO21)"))
 (via (at 150.855 117.425) (size 0.6) (drill 0.3) (layers "F.Cu" "B.Cu") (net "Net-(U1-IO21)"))
 (segment (start 156.93 123.5) (end 150.855 117.425) (width 0.2) (layer "B.Cu") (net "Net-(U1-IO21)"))
 (segment (start 161.5 123.5) (end 156.93 123.5) (width 0.2) (layer "B.Cu") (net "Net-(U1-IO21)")))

